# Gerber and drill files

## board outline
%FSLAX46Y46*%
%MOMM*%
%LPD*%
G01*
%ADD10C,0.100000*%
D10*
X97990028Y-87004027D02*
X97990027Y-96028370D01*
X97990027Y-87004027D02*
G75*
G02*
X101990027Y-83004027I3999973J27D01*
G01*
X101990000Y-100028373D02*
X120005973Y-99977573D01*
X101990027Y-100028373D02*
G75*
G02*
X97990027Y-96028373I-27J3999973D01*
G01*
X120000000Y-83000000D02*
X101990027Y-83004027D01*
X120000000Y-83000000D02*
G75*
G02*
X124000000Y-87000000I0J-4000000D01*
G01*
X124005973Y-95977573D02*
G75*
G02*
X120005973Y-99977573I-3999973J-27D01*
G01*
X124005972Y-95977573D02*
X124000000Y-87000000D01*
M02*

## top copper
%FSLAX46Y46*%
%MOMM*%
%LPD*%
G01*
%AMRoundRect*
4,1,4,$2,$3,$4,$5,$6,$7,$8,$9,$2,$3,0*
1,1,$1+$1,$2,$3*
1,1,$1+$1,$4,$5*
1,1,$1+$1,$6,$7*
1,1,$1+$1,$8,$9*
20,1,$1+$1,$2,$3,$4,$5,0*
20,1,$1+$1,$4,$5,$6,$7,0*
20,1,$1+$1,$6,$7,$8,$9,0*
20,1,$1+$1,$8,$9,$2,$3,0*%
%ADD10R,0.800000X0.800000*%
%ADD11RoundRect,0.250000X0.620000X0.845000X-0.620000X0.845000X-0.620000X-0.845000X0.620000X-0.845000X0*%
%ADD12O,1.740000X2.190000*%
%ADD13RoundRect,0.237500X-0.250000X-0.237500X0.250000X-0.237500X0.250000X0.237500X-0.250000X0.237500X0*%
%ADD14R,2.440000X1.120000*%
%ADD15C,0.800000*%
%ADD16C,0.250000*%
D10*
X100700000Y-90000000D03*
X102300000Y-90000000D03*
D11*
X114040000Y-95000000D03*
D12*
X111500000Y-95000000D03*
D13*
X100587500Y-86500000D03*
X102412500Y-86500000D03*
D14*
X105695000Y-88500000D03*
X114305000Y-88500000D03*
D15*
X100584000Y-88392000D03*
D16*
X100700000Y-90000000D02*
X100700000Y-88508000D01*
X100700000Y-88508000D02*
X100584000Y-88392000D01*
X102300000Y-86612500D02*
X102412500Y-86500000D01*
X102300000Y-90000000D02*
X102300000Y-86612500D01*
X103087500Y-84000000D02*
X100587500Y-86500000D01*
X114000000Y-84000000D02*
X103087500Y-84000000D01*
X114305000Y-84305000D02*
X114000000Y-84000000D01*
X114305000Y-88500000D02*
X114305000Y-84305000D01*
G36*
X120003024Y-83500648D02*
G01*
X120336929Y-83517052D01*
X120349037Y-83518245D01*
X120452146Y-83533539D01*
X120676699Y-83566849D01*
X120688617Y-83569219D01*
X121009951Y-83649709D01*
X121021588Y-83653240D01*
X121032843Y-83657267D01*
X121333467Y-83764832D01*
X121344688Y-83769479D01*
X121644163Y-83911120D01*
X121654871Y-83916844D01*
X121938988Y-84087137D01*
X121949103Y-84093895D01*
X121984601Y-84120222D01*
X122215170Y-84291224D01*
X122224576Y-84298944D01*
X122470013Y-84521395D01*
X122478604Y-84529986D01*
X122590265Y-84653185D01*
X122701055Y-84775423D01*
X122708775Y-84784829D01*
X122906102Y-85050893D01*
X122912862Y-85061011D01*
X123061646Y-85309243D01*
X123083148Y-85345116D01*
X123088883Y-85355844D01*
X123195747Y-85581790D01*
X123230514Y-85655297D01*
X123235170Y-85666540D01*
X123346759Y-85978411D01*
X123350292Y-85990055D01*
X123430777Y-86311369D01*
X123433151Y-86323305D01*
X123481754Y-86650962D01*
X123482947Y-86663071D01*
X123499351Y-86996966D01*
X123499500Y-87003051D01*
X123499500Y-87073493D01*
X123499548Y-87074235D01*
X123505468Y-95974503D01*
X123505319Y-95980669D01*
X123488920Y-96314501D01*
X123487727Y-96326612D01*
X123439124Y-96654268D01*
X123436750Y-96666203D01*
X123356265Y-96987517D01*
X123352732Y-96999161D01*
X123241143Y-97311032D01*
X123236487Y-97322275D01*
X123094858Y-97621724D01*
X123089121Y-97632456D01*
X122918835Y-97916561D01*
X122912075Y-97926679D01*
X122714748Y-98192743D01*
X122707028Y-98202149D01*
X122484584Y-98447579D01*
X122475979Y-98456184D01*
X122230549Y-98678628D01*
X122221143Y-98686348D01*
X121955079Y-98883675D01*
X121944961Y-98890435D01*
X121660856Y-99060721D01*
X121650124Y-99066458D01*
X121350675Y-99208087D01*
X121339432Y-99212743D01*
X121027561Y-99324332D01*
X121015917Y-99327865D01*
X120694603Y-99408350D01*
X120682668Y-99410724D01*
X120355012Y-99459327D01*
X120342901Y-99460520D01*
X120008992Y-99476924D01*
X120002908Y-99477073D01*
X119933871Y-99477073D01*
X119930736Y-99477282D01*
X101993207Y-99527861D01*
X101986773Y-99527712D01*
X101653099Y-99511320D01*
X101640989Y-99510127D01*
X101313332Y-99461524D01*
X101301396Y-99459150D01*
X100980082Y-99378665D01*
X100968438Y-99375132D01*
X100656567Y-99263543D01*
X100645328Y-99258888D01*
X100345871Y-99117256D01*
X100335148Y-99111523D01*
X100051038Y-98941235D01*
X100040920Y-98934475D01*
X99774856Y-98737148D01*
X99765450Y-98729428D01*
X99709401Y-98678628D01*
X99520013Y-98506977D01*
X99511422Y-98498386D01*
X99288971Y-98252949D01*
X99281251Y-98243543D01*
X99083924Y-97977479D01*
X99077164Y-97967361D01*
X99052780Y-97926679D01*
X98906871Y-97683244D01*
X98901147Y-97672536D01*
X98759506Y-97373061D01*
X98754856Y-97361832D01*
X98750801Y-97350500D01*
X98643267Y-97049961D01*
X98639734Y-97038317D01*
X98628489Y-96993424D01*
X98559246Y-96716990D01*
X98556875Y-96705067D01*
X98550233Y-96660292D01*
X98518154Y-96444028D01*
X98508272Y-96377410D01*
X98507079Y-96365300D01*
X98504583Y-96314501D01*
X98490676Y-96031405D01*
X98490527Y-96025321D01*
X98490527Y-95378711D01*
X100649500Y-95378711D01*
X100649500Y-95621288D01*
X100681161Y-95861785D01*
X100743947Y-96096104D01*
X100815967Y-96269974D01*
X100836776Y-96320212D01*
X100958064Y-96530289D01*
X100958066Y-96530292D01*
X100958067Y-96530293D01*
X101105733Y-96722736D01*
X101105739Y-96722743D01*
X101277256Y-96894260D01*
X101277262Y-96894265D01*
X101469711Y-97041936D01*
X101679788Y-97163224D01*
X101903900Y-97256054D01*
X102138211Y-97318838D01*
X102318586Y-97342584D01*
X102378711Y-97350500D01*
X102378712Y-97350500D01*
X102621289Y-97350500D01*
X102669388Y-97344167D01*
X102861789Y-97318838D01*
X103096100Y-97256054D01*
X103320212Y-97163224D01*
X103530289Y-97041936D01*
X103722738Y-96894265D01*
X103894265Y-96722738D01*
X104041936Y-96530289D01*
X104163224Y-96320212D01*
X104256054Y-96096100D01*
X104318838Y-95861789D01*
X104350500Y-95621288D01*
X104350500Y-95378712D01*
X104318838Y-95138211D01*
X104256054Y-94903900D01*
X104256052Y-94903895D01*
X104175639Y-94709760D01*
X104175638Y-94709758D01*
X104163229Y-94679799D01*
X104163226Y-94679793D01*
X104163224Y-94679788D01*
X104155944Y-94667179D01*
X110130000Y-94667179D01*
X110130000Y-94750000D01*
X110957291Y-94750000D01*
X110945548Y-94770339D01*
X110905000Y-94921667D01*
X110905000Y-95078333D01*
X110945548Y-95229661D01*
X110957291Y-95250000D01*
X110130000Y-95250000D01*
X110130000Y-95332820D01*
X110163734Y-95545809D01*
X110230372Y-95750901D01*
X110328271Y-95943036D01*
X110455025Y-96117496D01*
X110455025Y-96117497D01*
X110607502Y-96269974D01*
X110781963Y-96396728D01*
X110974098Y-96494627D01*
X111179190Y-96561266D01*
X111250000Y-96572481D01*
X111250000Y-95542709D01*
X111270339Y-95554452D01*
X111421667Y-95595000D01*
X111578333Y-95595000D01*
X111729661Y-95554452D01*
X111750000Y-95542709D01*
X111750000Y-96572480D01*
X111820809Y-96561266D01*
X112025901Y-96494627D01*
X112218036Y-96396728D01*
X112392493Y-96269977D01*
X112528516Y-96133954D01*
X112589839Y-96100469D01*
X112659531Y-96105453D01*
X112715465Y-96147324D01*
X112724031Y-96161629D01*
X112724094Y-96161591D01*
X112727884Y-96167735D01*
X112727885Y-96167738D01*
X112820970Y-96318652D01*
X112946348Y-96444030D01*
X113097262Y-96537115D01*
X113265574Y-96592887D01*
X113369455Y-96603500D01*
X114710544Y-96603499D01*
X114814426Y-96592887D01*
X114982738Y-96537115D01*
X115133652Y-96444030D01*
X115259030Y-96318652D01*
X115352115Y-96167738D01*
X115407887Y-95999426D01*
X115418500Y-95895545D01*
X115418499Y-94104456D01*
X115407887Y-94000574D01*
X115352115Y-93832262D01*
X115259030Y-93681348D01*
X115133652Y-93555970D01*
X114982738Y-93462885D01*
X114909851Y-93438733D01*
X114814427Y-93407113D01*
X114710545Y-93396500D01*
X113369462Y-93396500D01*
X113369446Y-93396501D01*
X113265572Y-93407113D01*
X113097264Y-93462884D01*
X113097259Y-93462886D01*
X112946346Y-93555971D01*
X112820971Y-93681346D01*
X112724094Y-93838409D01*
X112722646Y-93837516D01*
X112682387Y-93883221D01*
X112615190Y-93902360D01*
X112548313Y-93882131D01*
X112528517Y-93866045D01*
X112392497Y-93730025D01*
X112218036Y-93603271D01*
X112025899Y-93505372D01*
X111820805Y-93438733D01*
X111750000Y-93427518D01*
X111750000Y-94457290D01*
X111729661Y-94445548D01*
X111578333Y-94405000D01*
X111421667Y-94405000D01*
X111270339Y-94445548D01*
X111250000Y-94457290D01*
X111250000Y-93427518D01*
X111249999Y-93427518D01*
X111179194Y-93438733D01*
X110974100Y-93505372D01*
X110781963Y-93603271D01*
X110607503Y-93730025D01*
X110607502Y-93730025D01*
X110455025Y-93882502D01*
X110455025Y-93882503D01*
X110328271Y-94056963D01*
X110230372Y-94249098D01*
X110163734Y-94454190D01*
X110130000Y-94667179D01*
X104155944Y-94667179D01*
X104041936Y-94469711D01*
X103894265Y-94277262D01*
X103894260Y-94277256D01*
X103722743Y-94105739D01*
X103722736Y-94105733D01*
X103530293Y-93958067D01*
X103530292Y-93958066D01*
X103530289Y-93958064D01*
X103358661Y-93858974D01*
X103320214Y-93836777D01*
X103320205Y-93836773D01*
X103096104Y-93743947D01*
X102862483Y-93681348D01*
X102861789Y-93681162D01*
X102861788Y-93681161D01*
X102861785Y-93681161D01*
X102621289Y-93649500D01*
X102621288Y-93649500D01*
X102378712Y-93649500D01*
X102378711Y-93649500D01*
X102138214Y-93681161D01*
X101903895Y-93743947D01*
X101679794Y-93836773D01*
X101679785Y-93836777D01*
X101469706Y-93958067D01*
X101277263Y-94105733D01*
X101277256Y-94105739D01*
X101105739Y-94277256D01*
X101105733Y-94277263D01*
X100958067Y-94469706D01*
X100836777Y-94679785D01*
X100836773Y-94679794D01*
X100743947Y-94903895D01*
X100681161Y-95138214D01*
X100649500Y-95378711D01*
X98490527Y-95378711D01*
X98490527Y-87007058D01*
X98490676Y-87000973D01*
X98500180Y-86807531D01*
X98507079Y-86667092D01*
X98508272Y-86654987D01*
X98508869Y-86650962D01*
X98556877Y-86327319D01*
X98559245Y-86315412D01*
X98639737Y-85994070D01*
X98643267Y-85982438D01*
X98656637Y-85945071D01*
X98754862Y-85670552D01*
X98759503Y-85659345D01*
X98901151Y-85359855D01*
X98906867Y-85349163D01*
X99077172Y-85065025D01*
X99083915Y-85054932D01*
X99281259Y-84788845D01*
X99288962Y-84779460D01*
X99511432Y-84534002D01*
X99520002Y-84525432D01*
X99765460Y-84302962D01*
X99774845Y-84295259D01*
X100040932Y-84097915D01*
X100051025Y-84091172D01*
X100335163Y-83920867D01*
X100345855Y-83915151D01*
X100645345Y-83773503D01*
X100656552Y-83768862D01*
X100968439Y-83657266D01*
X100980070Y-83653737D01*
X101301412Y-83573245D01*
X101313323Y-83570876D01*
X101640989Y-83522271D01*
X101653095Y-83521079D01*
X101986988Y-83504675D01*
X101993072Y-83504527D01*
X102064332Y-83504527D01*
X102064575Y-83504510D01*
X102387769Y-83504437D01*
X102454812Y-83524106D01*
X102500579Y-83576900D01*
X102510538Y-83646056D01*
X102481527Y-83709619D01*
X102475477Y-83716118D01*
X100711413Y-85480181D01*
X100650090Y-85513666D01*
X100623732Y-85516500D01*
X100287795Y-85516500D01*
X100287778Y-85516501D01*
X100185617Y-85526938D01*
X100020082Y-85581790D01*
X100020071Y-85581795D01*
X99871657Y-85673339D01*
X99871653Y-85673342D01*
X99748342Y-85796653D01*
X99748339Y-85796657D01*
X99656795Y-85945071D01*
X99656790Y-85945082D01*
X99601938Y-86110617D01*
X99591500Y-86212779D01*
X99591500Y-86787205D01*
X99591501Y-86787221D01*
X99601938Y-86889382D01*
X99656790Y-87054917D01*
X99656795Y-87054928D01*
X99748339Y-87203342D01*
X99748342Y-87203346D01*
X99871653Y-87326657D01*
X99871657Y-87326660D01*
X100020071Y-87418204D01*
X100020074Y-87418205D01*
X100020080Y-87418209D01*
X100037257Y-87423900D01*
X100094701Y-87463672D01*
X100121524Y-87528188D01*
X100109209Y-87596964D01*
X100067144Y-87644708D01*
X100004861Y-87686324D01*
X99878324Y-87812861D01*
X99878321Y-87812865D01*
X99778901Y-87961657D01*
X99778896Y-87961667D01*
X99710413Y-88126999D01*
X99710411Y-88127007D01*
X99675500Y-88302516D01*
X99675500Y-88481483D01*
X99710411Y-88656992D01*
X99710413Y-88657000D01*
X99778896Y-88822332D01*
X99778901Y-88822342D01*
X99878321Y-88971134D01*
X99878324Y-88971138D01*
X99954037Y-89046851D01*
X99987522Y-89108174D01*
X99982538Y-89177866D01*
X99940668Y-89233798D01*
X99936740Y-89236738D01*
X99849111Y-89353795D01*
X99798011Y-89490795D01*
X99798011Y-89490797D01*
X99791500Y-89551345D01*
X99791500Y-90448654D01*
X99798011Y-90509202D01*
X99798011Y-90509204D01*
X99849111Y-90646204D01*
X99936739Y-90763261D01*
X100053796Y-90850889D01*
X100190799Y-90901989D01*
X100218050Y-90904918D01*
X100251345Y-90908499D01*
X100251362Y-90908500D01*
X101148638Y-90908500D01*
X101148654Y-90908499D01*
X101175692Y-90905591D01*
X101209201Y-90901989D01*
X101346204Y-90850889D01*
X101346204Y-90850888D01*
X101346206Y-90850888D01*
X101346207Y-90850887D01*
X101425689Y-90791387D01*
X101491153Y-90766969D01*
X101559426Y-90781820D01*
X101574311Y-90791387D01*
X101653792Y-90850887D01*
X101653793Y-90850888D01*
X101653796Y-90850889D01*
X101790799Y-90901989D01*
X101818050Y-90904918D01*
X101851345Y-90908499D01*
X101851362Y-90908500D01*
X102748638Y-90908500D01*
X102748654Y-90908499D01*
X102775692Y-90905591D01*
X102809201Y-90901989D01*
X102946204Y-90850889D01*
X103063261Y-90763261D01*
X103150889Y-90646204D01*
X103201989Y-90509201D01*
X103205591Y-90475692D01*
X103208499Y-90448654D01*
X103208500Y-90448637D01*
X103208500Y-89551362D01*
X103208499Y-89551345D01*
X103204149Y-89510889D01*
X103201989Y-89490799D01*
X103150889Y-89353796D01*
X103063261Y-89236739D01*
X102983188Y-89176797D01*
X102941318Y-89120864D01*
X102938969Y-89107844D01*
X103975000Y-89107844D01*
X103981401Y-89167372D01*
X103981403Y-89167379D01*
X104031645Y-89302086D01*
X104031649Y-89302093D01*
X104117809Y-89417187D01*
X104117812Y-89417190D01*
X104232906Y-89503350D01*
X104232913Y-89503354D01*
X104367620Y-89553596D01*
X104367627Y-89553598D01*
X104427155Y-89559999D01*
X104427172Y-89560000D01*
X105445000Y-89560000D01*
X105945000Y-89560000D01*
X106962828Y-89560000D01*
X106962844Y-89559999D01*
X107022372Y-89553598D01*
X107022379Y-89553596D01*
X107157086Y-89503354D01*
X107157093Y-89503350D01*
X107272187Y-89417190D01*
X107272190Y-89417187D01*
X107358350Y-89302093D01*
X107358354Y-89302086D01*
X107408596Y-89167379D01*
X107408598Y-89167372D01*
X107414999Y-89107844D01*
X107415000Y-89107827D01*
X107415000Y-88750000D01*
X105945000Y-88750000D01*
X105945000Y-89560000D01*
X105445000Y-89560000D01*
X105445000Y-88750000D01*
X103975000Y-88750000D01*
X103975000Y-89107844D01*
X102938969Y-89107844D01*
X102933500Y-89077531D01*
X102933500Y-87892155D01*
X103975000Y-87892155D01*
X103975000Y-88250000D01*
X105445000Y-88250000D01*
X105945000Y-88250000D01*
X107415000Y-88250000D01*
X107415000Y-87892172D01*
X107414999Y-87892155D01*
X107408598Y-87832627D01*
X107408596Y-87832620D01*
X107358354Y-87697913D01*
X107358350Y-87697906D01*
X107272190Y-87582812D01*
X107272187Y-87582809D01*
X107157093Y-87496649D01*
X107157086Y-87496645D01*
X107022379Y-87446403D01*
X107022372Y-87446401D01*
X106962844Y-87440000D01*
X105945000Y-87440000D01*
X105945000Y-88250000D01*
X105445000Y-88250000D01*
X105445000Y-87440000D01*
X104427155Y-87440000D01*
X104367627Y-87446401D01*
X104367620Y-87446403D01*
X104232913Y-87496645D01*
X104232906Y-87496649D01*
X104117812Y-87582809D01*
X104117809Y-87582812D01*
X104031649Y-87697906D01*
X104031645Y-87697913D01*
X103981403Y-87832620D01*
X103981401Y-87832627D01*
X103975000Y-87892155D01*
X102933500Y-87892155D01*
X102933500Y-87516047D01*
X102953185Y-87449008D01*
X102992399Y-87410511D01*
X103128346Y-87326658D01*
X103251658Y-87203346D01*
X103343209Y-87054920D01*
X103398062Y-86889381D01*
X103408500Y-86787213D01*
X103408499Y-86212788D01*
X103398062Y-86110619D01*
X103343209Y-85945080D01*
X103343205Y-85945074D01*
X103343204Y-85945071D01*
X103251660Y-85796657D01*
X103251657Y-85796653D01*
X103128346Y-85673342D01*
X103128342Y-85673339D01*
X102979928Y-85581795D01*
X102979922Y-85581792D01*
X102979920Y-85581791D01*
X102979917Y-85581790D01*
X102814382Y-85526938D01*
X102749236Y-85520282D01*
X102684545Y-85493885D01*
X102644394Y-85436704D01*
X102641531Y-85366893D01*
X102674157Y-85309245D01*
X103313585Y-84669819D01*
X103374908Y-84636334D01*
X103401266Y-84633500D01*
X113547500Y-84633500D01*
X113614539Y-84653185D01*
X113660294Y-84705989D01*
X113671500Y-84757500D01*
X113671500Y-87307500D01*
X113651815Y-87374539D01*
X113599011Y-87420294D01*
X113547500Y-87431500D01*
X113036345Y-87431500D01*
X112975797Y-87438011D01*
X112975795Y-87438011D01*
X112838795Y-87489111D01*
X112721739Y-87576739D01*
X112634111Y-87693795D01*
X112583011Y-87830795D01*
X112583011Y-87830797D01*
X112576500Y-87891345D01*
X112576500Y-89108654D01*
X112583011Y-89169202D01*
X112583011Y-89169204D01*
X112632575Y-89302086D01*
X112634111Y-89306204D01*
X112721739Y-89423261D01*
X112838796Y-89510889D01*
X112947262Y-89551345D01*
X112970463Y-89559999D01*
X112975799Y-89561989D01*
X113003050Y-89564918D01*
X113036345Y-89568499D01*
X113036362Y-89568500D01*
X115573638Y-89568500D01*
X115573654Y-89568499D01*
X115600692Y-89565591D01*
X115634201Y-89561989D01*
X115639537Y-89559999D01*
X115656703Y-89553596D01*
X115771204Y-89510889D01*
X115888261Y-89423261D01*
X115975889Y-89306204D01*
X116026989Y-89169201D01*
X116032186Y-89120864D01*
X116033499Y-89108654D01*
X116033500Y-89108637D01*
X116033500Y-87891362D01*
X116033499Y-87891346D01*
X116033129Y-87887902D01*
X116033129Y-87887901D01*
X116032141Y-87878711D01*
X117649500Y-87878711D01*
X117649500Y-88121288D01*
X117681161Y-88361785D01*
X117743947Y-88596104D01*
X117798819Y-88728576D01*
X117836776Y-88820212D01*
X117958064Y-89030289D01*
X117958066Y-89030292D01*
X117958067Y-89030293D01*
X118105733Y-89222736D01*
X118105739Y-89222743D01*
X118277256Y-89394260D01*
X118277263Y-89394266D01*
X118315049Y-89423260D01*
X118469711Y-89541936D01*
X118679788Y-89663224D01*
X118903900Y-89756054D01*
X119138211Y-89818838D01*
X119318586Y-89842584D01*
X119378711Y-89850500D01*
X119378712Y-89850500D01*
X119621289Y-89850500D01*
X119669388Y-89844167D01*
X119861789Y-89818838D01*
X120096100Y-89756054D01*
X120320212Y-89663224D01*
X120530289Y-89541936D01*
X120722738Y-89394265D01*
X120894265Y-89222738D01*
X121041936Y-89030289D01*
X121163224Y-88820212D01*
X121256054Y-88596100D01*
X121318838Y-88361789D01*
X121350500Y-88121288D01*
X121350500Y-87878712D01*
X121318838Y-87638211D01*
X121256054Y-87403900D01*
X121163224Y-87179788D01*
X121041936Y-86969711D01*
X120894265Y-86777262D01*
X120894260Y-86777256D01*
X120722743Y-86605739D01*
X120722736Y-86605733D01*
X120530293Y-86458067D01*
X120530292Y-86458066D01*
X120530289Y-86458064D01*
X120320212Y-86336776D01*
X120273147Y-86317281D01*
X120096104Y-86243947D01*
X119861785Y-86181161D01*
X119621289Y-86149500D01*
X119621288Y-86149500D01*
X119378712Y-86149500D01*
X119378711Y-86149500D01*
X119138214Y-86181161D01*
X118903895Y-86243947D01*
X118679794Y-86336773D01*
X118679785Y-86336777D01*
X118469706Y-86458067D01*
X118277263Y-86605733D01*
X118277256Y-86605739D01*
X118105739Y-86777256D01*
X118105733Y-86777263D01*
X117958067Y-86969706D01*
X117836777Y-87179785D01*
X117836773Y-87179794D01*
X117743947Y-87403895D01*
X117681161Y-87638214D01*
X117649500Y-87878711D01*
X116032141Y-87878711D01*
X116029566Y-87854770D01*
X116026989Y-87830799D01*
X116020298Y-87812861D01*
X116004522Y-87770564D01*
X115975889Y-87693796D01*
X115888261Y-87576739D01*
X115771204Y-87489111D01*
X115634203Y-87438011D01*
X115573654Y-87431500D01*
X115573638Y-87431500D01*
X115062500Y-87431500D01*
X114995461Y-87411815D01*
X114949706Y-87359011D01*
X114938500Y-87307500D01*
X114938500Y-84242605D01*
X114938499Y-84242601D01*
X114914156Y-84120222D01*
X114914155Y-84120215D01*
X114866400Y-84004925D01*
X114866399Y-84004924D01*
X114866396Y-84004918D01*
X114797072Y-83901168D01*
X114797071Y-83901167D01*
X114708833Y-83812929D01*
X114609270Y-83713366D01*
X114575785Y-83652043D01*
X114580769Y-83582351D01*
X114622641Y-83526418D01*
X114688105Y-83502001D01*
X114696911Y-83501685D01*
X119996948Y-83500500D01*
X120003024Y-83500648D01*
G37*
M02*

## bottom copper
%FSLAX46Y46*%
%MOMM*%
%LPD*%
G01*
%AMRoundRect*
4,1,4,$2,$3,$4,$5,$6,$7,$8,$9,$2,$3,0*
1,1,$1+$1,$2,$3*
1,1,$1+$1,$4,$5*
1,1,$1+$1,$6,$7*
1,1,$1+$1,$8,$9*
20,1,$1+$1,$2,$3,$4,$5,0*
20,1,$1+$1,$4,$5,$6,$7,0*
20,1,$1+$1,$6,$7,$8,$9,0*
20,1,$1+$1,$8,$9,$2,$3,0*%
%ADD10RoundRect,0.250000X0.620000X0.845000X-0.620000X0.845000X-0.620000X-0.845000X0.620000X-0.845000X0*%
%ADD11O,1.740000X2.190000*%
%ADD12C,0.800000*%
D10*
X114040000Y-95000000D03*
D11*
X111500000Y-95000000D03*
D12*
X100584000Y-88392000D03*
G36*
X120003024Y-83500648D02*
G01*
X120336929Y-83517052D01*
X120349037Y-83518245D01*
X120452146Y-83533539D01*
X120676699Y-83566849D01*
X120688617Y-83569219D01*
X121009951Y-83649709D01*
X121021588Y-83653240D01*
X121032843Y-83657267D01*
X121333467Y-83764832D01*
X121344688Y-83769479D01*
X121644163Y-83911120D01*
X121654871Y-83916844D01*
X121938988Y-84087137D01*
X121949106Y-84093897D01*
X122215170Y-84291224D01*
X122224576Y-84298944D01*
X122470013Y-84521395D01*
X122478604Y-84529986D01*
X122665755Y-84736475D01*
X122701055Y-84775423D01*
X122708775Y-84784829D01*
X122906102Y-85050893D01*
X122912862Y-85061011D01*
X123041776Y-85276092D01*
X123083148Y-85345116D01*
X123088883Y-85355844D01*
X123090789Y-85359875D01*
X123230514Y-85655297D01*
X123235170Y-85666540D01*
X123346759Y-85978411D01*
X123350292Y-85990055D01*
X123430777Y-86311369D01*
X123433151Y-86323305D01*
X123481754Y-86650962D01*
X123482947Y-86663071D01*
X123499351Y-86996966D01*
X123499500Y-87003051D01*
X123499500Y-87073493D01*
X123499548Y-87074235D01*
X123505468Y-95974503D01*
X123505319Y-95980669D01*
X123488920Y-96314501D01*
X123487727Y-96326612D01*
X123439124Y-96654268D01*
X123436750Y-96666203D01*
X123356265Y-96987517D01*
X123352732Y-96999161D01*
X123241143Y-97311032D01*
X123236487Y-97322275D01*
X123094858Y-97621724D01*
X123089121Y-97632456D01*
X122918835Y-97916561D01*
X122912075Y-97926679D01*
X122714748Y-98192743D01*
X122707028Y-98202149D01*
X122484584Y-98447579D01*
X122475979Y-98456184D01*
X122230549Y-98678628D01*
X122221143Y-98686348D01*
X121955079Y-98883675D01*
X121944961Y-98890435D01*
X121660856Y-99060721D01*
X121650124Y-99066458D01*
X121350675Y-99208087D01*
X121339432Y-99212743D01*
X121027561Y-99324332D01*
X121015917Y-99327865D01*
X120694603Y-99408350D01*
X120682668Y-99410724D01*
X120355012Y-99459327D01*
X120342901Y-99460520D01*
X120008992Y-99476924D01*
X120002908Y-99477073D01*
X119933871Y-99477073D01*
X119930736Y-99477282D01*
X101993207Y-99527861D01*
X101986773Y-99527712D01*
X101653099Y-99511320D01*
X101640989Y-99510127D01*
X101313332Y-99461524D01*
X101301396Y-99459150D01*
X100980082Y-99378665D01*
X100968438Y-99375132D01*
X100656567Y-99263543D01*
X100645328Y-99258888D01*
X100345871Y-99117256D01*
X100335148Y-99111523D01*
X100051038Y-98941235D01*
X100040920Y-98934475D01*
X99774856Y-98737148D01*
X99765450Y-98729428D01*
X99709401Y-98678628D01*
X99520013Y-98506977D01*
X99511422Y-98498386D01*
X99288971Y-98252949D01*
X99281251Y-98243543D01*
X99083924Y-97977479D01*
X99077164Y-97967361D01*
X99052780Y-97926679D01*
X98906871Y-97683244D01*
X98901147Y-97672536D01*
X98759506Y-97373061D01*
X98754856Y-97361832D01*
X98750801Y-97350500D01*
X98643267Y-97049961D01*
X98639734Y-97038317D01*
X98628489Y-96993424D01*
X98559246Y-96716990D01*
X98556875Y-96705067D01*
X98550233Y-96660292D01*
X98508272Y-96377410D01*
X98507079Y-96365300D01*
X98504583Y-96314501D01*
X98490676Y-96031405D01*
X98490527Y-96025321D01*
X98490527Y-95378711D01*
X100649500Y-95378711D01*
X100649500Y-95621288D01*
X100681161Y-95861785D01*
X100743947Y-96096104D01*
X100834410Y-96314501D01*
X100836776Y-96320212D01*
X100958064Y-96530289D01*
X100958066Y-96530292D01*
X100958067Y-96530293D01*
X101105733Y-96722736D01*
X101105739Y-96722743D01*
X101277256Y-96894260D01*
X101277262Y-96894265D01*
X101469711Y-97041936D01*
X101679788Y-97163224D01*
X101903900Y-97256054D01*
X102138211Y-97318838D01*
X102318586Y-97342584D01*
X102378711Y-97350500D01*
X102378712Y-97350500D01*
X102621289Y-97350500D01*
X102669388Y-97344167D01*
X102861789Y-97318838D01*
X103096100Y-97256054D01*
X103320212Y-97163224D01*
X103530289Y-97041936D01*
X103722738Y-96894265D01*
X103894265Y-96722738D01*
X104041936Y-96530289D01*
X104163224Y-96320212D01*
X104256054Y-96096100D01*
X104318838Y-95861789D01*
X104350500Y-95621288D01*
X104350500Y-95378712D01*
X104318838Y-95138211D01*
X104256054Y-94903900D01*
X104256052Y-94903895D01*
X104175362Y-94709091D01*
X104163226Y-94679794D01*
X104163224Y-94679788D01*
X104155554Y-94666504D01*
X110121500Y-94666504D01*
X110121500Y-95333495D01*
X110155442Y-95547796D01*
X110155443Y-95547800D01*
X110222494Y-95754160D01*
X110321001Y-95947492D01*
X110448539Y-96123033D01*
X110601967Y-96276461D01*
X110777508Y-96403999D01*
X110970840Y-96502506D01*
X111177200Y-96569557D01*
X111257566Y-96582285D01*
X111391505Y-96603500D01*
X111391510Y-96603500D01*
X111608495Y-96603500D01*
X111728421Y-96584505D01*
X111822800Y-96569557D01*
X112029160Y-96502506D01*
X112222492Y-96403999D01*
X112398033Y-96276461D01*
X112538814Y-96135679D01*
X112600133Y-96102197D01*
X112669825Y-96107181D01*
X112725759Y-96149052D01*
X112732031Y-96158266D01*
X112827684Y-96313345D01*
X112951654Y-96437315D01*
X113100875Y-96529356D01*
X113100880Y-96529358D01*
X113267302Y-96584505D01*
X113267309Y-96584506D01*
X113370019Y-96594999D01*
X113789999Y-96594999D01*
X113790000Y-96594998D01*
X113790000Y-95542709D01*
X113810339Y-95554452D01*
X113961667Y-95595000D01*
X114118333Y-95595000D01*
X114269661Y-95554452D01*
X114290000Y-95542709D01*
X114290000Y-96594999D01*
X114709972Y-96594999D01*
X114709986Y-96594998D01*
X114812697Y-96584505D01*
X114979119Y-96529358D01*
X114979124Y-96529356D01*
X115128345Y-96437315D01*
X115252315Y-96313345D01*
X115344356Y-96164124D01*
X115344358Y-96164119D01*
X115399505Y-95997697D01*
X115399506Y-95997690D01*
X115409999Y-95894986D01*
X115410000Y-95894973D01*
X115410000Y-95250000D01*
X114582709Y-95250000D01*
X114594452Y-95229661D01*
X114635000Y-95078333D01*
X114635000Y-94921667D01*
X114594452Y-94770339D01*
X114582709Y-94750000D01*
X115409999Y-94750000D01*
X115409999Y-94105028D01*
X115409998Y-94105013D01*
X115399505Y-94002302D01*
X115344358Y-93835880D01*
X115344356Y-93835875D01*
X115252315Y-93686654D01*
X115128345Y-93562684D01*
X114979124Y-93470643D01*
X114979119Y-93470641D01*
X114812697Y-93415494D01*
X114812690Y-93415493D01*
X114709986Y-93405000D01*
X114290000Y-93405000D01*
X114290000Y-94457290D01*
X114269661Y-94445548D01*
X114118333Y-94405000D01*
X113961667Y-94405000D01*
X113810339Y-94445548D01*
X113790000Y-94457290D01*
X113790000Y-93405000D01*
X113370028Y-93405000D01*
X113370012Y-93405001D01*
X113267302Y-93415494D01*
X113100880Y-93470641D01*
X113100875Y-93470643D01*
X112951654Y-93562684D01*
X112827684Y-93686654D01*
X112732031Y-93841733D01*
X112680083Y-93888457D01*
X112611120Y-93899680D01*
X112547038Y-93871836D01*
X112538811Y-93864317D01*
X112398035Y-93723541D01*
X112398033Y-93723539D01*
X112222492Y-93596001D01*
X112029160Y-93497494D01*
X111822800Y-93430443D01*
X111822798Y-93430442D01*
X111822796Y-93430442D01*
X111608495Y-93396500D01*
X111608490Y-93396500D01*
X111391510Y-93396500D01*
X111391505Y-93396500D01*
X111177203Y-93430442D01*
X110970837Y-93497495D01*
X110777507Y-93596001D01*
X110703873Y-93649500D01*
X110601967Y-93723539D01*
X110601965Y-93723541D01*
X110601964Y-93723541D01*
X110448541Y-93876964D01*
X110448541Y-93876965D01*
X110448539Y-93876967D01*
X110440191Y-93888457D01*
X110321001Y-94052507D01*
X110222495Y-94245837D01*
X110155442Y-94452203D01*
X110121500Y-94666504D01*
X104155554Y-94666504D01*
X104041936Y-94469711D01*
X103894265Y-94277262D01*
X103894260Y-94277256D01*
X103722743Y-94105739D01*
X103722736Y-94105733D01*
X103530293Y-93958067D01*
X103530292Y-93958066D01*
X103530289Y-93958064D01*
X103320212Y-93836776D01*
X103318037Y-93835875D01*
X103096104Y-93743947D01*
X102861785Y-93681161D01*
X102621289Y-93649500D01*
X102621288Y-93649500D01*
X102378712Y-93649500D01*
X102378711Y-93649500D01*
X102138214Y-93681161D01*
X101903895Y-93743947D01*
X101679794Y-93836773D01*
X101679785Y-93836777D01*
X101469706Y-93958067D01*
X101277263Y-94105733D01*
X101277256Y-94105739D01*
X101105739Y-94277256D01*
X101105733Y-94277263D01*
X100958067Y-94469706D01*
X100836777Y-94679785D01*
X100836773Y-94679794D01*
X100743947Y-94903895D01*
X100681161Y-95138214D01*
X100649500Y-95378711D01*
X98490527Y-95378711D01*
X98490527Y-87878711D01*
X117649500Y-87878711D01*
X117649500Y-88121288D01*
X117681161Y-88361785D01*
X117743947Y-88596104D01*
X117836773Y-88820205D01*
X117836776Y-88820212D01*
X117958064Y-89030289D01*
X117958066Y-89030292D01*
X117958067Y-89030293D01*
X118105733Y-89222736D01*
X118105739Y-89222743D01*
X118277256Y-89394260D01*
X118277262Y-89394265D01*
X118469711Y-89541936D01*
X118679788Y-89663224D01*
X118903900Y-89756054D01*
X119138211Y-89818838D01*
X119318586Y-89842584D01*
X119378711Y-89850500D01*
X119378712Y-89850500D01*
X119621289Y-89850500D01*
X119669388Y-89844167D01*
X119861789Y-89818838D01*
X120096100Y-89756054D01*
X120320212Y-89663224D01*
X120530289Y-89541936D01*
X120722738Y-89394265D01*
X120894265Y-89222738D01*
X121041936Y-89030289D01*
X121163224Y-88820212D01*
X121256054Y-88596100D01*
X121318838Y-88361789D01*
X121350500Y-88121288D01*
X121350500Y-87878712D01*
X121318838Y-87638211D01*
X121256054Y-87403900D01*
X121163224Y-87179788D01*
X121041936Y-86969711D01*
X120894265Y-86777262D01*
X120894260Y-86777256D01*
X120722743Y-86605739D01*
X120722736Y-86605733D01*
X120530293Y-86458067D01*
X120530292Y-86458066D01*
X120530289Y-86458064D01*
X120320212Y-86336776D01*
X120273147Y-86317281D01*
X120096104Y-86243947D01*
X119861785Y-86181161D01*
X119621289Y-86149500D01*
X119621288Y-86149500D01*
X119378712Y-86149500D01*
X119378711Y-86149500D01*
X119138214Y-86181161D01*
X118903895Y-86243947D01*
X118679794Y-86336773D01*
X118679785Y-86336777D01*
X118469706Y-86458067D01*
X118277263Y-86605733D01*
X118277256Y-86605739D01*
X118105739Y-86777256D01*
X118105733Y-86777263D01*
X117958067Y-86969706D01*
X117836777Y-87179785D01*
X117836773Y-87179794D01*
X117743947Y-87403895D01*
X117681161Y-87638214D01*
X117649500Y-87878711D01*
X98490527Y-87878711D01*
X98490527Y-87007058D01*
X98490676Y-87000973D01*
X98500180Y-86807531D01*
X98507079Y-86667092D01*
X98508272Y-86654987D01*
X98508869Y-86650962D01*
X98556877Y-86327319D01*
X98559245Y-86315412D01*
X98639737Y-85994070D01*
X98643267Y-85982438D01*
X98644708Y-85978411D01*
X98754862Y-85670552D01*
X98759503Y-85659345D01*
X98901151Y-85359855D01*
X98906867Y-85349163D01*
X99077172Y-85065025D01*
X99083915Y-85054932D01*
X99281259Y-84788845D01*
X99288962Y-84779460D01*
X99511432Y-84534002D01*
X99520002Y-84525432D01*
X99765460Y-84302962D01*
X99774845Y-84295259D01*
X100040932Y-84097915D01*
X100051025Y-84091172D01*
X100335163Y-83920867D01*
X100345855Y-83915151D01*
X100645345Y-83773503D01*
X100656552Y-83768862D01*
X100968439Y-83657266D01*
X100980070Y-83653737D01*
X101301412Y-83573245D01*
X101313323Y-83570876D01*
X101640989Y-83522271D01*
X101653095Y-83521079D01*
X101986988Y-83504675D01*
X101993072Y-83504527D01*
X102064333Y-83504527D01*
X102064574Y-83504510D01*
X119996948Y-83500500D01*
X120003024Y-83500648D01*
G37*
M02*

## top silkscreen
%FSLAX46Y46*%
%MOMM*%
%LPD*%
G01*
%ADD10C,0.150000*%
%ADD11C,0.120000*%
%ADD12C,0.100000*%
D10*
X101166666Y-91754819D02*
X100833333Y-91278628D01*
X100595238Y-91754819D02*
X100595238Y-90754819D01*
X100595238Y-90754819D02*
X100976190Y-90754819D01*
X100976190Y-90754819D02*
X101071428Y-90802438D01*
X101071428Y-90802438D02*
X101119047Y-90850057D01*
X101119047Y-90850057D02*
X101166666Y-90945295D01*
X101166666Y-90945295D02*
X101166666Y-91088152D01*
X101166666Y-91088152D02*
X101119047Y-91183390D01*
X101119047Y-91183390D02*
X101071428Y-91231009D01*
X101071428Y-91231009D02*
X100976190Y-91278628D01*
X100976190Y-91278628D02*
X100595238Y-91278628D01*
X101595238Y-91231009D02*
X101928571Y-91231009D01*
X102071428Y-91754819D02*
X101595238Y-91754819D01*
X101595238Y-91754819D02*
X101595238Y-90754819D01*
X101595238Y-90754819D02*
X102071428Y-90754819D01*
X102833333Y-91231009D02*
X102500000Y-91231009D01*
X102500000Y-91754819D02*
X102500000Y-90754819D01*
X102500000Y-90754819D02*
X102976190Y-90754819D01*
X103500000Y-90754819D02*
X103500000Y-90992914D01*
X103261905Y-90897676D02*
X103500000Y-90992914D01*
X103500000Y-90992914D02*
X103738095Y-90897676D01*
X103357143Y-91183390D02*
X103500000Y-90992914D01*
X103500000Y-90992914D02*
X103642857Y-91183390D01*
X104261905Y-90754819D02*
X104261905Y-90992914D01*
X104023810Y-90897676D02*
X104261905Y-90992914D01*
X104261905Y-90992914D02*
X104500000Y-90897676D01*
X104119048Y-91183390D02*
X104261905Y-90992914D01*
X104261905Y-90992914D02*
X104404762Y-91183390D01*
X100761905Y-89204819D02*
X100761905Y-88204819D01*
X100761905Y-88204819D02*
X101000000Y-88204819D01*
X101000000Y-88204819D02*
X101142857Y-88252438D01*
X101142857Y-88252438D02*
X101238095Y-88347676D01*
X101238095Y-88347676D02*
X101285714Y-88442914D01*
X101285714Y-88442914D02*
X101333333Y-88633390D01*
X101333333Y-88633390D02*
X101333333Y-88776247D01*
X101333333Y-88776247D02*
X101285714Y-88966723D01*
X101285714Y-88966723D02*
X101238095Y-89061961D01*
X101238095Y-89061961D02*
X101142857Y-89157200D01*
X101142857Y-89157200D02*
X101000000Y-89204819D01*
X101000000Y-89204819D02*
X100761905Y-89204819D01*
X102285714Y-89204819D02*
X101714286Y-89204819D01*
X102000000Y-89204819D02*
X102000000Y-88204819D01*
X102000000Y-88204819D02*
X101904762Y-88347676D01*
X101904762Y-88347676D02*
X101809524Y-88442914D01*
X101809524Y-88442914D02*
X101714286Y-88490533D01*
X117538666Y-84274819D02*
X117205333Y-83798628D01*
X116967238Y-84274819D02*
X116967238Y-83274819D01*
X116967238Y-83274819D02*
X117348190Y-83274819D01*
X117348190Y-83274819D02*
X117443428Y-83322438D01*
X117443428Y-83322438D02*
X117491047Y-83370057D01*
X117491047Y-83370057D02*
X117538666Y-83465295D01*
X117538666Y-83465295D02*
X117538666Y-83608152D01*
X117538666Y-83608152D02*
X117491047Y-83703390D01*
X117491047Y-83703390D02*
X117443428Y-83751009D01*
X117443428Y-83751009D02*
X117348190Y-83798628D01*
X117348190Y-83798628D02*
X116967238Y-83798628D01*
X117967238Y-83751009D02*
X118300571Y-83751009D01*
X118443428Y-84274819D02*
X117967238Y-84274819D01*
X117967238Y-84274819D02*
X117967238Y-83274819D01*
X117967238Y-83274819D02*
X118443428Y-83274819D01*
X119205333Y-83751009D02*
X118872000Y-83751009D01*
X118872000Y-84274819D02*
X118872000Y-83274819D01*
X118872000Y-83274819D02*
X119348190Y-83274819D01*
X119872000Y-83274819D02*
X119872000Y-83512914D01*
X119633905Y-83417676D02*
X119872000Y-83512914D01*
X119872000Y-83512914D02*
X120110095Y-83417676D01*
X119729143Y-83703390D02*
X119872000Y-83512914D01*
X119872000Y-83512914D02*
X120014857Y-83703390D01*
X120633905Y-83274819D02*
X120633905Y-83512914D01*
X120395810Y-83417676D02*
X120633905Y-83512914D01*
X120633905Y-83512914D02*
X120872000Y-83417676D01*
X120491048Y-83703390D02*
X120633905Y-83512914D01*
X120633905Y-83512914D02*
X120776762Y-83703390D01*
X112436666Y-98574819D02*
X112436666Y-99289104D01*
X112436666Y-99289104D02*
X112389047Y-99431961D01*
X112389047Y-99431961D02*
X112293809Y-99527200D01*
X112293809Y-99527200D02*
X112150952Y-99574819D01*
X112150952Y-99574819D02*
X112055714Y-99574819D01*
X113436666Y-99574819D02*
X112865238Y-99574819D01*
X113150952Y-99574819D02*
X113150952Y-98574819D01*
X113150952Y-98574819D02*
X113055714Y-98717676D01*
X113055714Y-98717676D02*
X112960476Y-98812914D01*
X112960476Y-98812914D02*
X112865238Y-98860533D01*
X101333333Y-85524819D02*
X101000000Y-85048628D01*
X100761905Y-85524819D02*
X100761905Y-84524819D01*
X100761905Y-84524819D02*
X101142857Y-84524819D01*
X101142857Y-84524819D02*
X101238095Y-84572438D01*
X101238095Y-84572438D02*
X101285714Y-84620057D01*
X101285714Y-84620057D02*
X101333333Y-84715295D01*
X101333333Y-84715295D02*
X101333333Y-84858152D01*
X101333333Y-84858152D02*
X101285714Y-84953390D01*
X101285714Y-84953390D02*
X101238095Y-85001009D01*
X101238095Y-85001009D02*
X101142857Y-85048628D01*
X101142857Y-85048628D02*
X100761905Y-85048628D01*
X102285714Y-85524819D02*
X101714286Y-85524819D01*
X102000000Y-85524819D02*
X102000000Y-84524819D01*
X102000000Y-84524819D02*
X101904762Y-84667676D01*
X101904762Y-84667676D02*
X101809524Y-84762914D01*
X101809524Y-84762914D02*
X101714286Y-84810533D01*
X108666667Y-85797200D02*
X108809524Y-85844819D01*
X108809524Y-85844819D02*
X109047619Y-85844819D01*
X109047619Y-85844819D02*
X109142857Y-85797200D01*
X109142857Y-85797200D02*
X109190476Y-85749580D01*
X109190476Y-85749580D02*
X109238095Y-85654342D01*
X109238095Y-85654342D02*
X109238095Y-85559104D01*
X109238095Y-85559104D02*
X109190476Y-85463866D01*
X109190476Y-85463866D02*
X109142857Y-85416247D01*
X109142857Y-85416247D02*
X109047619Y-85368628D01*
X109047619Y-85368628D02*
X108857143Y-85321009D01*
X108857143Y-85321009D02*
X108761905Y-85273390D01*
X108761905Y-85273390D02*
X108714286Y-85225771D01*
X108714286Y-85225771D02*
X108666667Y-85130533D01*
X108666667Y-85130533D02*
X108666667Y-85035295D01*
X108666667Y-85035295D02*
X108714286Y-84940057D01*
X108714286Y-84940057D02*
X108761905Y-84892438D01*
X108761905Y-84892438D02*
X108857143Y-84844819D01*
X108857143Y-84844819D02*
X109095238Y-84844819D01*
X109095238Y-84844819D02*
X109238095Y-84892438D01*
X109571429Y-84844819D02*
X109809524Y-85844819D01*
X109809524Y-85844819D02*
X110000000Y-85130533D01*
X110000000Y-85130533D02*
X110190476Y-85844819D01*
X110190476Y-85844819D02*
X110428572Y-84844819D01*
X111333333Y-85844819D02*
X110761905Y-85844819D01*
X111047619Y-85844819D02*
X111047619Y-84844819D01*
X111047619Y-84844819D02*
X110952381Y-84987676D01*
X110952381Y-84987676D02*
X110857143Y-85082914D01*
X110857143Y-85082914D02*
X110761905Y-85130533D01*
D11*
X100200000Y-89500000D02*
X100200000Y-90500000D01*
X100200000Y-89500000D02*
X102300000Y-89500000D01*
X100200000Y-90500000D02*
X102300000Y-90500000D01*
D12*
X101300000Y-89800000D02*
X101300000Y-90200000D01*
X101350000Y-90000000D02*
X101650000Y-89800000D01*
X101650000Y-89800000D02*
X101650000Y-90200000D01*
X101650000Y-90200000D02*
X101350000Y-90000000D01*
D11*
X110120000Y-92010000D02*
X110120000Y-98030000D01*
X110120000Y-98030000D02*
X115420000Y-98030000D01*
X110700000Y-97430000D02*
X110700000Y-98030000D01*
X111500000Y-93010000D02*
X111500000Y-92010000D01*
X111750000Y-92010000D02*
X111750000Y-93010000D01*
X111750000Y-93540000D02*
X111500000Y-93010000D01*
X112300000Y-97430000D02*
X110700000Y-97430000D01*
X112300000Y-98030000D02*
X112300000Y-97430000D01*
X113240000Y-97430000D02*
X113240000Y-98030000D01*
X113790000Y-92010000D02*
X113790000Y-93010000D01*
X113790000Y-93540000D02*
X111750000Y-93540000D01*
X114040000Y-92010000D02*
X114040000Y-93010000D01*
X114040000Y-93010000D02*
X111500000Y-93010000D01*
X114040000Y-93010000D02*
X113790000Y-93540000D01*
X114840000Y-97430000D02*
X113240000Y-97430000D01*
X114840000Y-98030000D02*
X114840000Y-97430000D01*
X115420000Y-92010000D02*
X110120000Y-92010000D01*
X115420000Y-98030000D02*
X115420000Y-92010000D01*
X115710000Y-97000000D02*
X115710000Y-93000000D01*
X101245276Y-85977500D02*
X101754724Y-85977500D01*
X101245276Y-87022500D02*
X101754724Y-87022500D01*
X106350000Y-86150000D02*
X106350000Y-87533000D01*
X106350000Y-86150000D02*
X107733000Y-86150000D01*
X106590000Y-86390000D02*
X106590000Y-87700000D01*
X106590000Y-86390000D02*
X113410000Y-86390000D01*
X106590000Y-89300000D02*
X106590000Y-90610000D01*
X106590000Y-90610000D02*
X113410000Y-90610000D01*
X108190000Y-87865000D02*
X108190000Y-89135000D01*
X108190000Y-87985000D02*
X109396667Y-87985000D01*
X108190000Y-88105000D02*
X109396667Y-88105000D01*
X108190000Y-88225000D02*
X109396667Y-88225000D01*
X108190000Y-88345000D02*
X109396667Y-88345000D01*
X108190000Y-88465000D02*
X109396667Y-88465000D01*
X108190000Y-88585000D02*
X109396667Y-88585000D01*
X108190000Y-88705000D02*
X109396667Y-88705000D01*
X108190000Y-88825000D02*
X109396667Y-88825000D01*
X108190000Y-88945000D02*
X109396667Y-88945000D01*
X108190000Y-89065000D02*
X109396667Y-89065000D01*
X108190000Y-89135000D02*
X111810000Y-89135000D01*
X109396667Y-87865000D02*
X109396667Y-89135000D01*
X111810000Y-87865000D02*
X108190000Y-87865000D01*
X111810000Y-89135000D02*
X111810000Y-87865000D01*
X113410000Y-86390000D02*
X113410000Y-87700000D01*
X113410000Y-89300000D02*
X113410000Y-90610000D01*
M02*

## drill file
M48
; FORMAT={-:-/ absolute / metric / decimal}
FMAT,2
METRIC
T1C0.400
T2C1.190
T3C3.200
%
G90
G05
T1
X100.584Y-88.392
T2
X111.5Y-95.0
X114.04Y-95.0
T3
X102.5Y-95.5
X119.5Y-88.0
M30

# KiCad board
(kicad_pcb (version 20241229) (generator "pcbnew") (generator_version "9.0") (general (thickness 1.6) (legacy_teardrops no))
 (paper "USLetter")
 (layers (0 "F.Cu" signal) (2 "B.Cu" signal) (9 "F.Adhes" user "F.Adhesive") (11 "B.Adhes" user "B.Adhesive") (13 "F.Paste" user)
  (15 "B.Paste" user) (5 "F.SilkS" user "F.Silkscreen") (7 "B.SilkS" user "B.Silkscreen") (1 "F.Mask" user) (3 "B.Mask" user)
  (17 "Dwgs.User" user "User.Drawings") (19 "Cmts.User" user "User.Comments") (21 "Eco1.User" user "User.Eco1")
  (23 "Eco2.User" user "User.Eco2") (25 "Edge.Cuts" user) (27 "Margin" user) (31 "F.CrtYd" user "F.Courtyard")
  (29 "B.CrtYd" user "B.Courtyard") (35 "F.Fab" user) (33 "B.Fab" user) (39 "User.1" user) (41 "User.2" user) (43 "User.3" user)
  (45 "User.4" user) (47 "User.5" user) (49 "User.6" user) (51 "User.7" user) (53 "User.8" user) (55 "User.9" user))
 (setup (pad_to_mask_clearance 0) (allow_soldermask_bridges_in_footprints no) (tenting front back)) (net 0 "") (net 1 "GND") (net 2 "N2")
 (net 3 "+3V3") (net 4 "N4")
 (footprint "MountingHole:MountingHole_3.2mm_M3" (layer "F.Cu") (at 102.5 95.5)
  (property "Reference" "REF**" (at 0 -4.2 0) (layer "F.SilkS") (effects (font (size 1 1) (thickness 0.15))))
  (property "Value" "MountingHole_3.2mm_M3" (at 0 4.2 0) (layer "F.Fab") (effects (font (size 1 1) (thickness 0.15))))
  (pad "" np_thru_hole circle (at 0 0) (size 3.2 3.2) (drill 3.2) (layers "*.Cu" "*.Mask")))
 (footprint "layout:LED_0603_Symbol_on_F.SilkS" (layer "F.Cu") (at 101.5 90)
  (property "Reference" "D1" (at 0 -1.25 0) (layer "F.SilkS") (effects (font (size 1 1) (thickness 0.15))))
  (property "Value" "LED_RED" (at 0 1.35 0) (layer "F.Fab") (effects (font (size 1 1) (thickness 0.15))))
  (fp_line (start -1.3 -0.5) (end -1.3 0.5) (stroke (width 0.12) (type solid)) (layer "F.SilkS"))
  (fp_line (start -1.3 -0.5) (end 0.8 -0.5) (stroke (width 0.12) (type solid)) (layer "F.SilkS"))
  (fp_line (start -1.3 0.5) (end 0.8 0.5) (stroke (width 0.12) (type solid)) (layer "F.SilkS"))
  (fp_line (start -0.2 -0.2) (end -0.2 0.2) (stroke (width 0.1) (type solid)) (layer "F.SilkS"))
  (fp_line (start -0.15 0) (end 0.15 -0.2) (stroke (width 0.1) (type solid)) (layer "F.SilkS"))
  (fp_line (start 0.15 -0.2) (end 0.15 0.2) (stroke (width 0.1) (type solid)) (layer "F.SilkS"))
  (fp_line (start 0.15 0.2) (end -0.15 0) (stroke (width 0.1) (type solid)) (layer "F.SilkS"))
  (pad "1" smd rect (at -0.8 0 180) (size 0.8 0.8) (layers "F.Cu" "F.Mask" "F.Paste") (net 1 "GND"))
  (pad "2" smd rect (at 0.8 0 180) (size 0.8 0.8) (layers "F.Cu" "F.Mask" "F.Paste") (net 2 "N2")))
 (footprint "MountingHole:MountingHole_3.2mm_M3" (layer "F.Cu") (at 119.5 88)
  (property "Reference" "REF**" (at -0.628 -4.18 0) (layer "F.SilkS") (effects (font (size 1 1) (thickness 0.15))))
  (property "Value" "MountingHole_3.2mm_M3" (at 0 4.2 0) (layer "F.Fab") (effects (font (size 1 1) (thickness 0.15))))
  (pad "" np_thru_hole circle (at 0 0) (size 3.2 3.2) (drill 3.2) (layers "*.Cu" "*.Mask")))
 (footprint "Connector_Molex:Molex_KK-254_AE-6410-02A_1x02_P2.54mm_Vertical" (layer "F.Cu") (at 114.04 95 180)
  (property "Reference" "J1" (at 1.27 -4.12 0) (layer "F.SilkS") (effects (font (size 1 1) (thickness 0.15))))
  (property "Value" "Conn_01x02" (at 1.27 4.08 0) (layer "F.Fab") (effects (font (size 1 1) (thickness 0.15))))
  (fp_line (start 3.92 2.99) (end 3.92 -3.03) (stroke (width 0.12) (type solid)) (layer "F.SilkS"))
  (fp_line (start 3.92 -3.03) (end -1.38 -3.03) (stroke (width 0.12) (type solid)) (layer "F.SilkS"))
  (fp_line (start 3.34 -2.43) (end 3.34 -3.03) (stroke (width 0.12) (type solid)) (layer "F.SilkS"))
  (fp_line (start 2.54 1.99) (end 2.54 2.99) (stroke (width 0.12) (type solid)) (layer "F.SilkS"))
  (fp_line (start 2.29 2.99) (end 2.29 1.99) (stroke (width 0.12) (type solid)) (layer "F.SilkS"))
  (fp_line (start 2.29 1.46) (end 2.54 1.99) (stroke (width 0.12) (type solid)) (layer "F.SilkS"))
  (fp_line (start 1.74 -2.43) (end 3.34 -2.43) (stroke (width 0.12) (type solid)) (layer "F.SilkS"))
  (fp_line (start 1.74 -3.03) (end 1.74 -2.43) (stroke (width 0.12) (type solid)) (layer "F.SilkS"))
  (fp_line (start 0.8 -2.43) (end 0.8 -3.03) (stroke (width 0.12) (type solid)) (layer "F.SilkS"))
  (fp_line (start 0.25 2.99) (end 0.25 1.99) (stroke (width 0.12) (type solid)) (layer "F.SilkS"))
  (fp_line (start 0.25 1.46) (end 2.29 1.46) (stroke (width 0.12) (type solid)) (layer "F.SilkS"))
  (fp_line (start 0 2.99) (end 0 1.99) (stroke (width 0.12) (type solid)) (layer "F.SilkS"))
  (fp_line (start 0 1.99) (end 2.54 1.99) (stroke (width 0.12) (type solid)) (layer "F.SilkS"))
  (fp_line (start 0 1.99) (end 0.25 1.46) (stroke (width 0.12) (type solid)) (layer "F.SilkS"))
  (fp_line (start -0.8 -2.43) (end 0.8 -2.43) (stroke (width 0.12) (type solid)) (layer "F.SilkS"))
  (fp_line (start -0.8 -3.03) (end -0.8 -2.43) (stroke (width 0.12) (type solid)) (layer "F.SilkS"))
  (fp_line (start -1.38 2.99) (end 3.92 2.99) (stroke (width 0.12) (type solid)) (layer "F.SilkS"))
  (fp_line (start -1.38 -3.03) (end -1.38 2.99) (stroke (width 0.12) (type solid)) (layer "F.SilkS"))
  (fp_line (start -1.67 -2) (end -1.67 2) (stroke (width 0.12) (type solid)) (layer "F.SilkS"))
  (pad "1" thru_hole roundrect (at 0 0 180) (size 1.74 2.19) (drill 1.19) (layers "*.Cu" "*.Mask") (remove_unused_layers no)
   (roundrect_rratio 0.143678) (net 1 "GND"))
  (pad "2" thru_hole oval (at 2.54 0 180) (size 1.74 2.19) (drill 1.19) (layers "*.Cu" "*.Mask") (remove_unused_layers no) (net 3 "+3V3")))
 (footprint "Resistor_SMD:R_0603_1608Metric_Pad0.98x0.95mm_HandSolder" (layer "F.Cu") (at 101.5 86.5)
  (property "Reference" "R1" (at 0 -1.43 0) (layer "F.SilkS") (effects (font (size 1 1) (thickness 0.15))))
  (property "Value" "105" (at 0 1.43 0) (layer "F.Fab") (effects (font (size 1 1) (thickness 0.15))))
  (fp_line (start -0.254724 -0.5225) (end 0.254724 -0.5225) (stroke (width 0.12) (type solid)) (layer "F.SilkS"))
  (fp_line (start -0.254724 0.5225) (end 0.254724 0.5225) (stroke (width 0.12) (type solid)) (layer "F.SilkS"))
  (pad "1" smd roundrect (at -0.9125 0) (size 0.975 0.95) (layers "F.Cu" "F.Mask" "F.Paste") (roundrect_rratio 0.25) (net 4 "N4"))
  (pad "2" smd roundrect (at 0.9125 0) (size 0.975 0.95) (layers "F.Cu" "F.Mask" "F.Paste") (roundrect_rratio 0.25) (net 2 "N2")))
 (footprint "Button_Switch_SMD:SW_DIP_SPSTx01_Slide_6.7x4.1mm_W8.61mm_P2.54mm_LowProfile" (layer "F.Cu") (at 110 88.5)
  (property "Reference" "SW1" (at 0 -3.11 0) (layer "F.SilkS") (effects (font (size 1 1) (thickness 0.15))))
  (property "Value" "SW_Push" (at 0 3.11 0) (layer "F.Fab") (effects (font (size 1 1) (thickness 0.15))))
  (fp_line (start -3.65 -2.35) (end -3.65 -0.967) (stroke (width 0.12) (type solid)) (layer "F.SilkS"))
  (fp_line (start -3.65 -2.35) (end -2.267 -2.35) (stroke (width 0.12) (type solid)) (layer "F.SilkS"))
  (fp_line (start -3.41 -2.11) (end -3.41 -0.8) (stroke (width 0.12) (type solid)) (layer "F.SilkS"))
  (fp_line (start -3.41 -2.11) (end 3.41 -2.11) (stroke (width 0.12) (type solid)) (layer "F.SilkS"))
  (fp_line (start -3.41 0.8) (end -3.41 2.11) (stroke (width 0.12) (type solid)) (layer "F.SilkS"))
  (fp_line (start -3.41 2.11) (end 3.41 2.11) (stroke (width 0.12) (type solid)) (layer "F.SilkS"))
  (fp_line (start -1.81 -0.635) (end -1.81 0.635) (stroke (width 0.12) (type solid)) (layer "F.SilkS"))
  (fp_line (start -1.81 -0.515) (end -0.603333 -0.515) (stroke (width 0.12) (type solid)) (layer "F.SilkS"))
  (fp_line (start -1.81 -0.395) (end -0.603333 -0.395) (stroke (width 0.12) (type solid)) (layer "F.SilkS"))
  (fp_line (start -1.81 -0.275) (end -0.603333 -0.275) (stroke (width 0.12) (type solid)) (layer "F.SilkS"))
  (fp_line (start -1.81 -0.155) (end -0.603333 -0.155) (stroke (width 0.12) (type solid)) (layer "F.SilkS"))
  (fp_line (start -1.81 -0.035) (end -0.603333 -0.035) (stroke (width 0.12) (type solid)) (layer "F.SilkS"))
  (fp_line (start -1.81 0.085) (end -0.603333 0.085) (stroke (width 0.12) (type solid)) (layer "F.SilkS"))
  (fp_line (start -1.81 0.205) (end -0.603333 0.205) (stroke (width 0.12) (type solid)) (layer "F.SilkS"))
  (fp_line (start -1.81 0.325) (end -0.603333 0.325) (stroke (width 0.12) (type solid)) (layer "F.SilkS"))
  (fp_line (start -1.81 0.445) (end -0.603333 0.445) (stroke (width 0.12) (type solid)) (layer "F.SilkS"))
  (fp_line (start -1.81 0.565) (end -0.603333 0.565) (stroke (width 0.12) (type solid)) (layer "F.SilkS"))
  (fp_line (start -1.81 0.635) (end 1.81 0.635) (stroke (width 0.12) (type solid)) (layer "F.SilkS"))
  (fp_line (start -0.603333 -0.635) (end -0.603333 0.635) (stroke (width 0.12) (type solid)) (layer "F.SilkS"))
  (fp_line (start 1.81 -0.635) (end -1.81 -0.635) (stroke (width 0.12) (type solid)) (layer "F.SilkS"))
  (fp_line (start 1.81 0.635) (end 1.81 -0.635) (stroke (width 0.12) (type solid)) (layer "F.SilkS"))
  (fp_line (start 3.41 -2.11) (end 3.41 -0.8) (stroke (width 0.12) (type solid)) (layer "F.SilkS"))
  (fp_line (start 3.41 0.8) (end 3.41 2.11) (stroke (width 0.12) (type solid)) (layer "F.SilkS"))
  (pad "1" smd rect (at -4.305 0) (size 2.44 1.12) (layers "F.Cu" "F.Mask" "F.Paste") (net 3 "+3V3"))
  (pad "2" smd rect (at 4.305 0) (size 2.44 1.12) (layers "F.Cu" "F.Mask" "F.Paste") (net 4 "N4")))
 (gr_line (start 97.990028 87.004027) (end 97.990027 96.02837) (stroke (width 0.1) (type default)) (layer "Edge.Cuts"))
 (gr_arc (start 97.990027 87.004027) (mid 99.1616 84.1756) (end 101.990027 83.004027) (stroke (width 0.1) (type default))
  (layer "Edge.Cuts"))
 (gr_line (start 101.99 100.028373) (end 120.005973 99.977573) (stroke (width 0.1) (type default)) (layer "Edge.Cuts"))
 (gr_arc (start 101.990027 100.028373) (mid 99.1616 98.8568) (end 97.990027 96.028373) (stroke (width 0.1) (type default))
  (layer "Edge.Cuts"))
 (gr_line (start 120 83) (end 101.990027 83.004027) (stroke (width 0.1) (type default)) (layer "Edge.Cuts"))
 (gr_arc (start 120 83) (mid 122.828427 84.171573) (end 124 87) (stroke (width 0.1) (type default)) (layer "Edge.Cuts"))
 (gr_arc (start 124.005973 95.977573) (mid 122.8344 98.806) (end 120.005973 99.977573) (stroke (width 0.1) (type default))
  (layer "Edge.Cuts"))
 (gr_line (start 124.005972 95.977573) (end 124 87) (stroke (width 0.1) (type default)) (layer "Edge.Cuts"))
 (segment (start 100.7 90) (end 100.7 88.508) (width 0.25) (layer "F.Cu") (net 1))
 (segment (start 100.7 88.508) (end 100.584 88.392) (width 0.25) (layer "F.Cu") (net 1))
 (via (at 100.584 88.392) (size 0.8) (drill 0.4) (layers "F.Cu" "B.Cu") (free yes) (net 1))
 (segment (start 102.3 86.6125) (end 102.4125 86.5) (width 0.25) (layer "F.Cu") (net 2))
 (segment (start 102.3 90) (end 102.3 86.6125) (width 0.25) (layer "F.Cu") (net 2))
 (segment (start 103.0875 84) (end 100.5875 86.5) (width 0.25) (layer "F.Cu") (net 4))
 (segment (start 114 84) (end 103.0875 84) (width 0.25) (layer "F.Cu") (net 4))
 (segment (start 114.305 84.305) (end 114 84) (width 0.25) (layer "F.Cu") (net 4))
 (segment (start 114.305 88.5) (end 114.305 84.305) (width 0.25) (layer "F.Cu") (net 4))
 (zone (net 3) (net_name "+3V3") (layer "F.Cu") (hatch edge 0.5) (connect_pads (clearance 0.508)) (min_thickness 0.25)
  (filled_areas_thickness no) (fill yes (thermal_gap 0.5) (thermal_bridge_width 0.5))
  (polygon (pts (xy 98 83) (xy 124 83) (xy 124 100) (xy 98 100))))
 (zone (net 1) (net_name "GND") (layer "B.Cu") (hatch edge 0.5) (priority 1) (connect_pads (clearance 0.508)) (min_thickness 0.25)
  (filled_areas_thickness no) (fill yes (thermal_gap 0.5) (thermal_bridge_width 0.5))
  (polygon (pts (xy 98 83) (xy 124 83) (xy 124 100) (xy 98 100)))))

